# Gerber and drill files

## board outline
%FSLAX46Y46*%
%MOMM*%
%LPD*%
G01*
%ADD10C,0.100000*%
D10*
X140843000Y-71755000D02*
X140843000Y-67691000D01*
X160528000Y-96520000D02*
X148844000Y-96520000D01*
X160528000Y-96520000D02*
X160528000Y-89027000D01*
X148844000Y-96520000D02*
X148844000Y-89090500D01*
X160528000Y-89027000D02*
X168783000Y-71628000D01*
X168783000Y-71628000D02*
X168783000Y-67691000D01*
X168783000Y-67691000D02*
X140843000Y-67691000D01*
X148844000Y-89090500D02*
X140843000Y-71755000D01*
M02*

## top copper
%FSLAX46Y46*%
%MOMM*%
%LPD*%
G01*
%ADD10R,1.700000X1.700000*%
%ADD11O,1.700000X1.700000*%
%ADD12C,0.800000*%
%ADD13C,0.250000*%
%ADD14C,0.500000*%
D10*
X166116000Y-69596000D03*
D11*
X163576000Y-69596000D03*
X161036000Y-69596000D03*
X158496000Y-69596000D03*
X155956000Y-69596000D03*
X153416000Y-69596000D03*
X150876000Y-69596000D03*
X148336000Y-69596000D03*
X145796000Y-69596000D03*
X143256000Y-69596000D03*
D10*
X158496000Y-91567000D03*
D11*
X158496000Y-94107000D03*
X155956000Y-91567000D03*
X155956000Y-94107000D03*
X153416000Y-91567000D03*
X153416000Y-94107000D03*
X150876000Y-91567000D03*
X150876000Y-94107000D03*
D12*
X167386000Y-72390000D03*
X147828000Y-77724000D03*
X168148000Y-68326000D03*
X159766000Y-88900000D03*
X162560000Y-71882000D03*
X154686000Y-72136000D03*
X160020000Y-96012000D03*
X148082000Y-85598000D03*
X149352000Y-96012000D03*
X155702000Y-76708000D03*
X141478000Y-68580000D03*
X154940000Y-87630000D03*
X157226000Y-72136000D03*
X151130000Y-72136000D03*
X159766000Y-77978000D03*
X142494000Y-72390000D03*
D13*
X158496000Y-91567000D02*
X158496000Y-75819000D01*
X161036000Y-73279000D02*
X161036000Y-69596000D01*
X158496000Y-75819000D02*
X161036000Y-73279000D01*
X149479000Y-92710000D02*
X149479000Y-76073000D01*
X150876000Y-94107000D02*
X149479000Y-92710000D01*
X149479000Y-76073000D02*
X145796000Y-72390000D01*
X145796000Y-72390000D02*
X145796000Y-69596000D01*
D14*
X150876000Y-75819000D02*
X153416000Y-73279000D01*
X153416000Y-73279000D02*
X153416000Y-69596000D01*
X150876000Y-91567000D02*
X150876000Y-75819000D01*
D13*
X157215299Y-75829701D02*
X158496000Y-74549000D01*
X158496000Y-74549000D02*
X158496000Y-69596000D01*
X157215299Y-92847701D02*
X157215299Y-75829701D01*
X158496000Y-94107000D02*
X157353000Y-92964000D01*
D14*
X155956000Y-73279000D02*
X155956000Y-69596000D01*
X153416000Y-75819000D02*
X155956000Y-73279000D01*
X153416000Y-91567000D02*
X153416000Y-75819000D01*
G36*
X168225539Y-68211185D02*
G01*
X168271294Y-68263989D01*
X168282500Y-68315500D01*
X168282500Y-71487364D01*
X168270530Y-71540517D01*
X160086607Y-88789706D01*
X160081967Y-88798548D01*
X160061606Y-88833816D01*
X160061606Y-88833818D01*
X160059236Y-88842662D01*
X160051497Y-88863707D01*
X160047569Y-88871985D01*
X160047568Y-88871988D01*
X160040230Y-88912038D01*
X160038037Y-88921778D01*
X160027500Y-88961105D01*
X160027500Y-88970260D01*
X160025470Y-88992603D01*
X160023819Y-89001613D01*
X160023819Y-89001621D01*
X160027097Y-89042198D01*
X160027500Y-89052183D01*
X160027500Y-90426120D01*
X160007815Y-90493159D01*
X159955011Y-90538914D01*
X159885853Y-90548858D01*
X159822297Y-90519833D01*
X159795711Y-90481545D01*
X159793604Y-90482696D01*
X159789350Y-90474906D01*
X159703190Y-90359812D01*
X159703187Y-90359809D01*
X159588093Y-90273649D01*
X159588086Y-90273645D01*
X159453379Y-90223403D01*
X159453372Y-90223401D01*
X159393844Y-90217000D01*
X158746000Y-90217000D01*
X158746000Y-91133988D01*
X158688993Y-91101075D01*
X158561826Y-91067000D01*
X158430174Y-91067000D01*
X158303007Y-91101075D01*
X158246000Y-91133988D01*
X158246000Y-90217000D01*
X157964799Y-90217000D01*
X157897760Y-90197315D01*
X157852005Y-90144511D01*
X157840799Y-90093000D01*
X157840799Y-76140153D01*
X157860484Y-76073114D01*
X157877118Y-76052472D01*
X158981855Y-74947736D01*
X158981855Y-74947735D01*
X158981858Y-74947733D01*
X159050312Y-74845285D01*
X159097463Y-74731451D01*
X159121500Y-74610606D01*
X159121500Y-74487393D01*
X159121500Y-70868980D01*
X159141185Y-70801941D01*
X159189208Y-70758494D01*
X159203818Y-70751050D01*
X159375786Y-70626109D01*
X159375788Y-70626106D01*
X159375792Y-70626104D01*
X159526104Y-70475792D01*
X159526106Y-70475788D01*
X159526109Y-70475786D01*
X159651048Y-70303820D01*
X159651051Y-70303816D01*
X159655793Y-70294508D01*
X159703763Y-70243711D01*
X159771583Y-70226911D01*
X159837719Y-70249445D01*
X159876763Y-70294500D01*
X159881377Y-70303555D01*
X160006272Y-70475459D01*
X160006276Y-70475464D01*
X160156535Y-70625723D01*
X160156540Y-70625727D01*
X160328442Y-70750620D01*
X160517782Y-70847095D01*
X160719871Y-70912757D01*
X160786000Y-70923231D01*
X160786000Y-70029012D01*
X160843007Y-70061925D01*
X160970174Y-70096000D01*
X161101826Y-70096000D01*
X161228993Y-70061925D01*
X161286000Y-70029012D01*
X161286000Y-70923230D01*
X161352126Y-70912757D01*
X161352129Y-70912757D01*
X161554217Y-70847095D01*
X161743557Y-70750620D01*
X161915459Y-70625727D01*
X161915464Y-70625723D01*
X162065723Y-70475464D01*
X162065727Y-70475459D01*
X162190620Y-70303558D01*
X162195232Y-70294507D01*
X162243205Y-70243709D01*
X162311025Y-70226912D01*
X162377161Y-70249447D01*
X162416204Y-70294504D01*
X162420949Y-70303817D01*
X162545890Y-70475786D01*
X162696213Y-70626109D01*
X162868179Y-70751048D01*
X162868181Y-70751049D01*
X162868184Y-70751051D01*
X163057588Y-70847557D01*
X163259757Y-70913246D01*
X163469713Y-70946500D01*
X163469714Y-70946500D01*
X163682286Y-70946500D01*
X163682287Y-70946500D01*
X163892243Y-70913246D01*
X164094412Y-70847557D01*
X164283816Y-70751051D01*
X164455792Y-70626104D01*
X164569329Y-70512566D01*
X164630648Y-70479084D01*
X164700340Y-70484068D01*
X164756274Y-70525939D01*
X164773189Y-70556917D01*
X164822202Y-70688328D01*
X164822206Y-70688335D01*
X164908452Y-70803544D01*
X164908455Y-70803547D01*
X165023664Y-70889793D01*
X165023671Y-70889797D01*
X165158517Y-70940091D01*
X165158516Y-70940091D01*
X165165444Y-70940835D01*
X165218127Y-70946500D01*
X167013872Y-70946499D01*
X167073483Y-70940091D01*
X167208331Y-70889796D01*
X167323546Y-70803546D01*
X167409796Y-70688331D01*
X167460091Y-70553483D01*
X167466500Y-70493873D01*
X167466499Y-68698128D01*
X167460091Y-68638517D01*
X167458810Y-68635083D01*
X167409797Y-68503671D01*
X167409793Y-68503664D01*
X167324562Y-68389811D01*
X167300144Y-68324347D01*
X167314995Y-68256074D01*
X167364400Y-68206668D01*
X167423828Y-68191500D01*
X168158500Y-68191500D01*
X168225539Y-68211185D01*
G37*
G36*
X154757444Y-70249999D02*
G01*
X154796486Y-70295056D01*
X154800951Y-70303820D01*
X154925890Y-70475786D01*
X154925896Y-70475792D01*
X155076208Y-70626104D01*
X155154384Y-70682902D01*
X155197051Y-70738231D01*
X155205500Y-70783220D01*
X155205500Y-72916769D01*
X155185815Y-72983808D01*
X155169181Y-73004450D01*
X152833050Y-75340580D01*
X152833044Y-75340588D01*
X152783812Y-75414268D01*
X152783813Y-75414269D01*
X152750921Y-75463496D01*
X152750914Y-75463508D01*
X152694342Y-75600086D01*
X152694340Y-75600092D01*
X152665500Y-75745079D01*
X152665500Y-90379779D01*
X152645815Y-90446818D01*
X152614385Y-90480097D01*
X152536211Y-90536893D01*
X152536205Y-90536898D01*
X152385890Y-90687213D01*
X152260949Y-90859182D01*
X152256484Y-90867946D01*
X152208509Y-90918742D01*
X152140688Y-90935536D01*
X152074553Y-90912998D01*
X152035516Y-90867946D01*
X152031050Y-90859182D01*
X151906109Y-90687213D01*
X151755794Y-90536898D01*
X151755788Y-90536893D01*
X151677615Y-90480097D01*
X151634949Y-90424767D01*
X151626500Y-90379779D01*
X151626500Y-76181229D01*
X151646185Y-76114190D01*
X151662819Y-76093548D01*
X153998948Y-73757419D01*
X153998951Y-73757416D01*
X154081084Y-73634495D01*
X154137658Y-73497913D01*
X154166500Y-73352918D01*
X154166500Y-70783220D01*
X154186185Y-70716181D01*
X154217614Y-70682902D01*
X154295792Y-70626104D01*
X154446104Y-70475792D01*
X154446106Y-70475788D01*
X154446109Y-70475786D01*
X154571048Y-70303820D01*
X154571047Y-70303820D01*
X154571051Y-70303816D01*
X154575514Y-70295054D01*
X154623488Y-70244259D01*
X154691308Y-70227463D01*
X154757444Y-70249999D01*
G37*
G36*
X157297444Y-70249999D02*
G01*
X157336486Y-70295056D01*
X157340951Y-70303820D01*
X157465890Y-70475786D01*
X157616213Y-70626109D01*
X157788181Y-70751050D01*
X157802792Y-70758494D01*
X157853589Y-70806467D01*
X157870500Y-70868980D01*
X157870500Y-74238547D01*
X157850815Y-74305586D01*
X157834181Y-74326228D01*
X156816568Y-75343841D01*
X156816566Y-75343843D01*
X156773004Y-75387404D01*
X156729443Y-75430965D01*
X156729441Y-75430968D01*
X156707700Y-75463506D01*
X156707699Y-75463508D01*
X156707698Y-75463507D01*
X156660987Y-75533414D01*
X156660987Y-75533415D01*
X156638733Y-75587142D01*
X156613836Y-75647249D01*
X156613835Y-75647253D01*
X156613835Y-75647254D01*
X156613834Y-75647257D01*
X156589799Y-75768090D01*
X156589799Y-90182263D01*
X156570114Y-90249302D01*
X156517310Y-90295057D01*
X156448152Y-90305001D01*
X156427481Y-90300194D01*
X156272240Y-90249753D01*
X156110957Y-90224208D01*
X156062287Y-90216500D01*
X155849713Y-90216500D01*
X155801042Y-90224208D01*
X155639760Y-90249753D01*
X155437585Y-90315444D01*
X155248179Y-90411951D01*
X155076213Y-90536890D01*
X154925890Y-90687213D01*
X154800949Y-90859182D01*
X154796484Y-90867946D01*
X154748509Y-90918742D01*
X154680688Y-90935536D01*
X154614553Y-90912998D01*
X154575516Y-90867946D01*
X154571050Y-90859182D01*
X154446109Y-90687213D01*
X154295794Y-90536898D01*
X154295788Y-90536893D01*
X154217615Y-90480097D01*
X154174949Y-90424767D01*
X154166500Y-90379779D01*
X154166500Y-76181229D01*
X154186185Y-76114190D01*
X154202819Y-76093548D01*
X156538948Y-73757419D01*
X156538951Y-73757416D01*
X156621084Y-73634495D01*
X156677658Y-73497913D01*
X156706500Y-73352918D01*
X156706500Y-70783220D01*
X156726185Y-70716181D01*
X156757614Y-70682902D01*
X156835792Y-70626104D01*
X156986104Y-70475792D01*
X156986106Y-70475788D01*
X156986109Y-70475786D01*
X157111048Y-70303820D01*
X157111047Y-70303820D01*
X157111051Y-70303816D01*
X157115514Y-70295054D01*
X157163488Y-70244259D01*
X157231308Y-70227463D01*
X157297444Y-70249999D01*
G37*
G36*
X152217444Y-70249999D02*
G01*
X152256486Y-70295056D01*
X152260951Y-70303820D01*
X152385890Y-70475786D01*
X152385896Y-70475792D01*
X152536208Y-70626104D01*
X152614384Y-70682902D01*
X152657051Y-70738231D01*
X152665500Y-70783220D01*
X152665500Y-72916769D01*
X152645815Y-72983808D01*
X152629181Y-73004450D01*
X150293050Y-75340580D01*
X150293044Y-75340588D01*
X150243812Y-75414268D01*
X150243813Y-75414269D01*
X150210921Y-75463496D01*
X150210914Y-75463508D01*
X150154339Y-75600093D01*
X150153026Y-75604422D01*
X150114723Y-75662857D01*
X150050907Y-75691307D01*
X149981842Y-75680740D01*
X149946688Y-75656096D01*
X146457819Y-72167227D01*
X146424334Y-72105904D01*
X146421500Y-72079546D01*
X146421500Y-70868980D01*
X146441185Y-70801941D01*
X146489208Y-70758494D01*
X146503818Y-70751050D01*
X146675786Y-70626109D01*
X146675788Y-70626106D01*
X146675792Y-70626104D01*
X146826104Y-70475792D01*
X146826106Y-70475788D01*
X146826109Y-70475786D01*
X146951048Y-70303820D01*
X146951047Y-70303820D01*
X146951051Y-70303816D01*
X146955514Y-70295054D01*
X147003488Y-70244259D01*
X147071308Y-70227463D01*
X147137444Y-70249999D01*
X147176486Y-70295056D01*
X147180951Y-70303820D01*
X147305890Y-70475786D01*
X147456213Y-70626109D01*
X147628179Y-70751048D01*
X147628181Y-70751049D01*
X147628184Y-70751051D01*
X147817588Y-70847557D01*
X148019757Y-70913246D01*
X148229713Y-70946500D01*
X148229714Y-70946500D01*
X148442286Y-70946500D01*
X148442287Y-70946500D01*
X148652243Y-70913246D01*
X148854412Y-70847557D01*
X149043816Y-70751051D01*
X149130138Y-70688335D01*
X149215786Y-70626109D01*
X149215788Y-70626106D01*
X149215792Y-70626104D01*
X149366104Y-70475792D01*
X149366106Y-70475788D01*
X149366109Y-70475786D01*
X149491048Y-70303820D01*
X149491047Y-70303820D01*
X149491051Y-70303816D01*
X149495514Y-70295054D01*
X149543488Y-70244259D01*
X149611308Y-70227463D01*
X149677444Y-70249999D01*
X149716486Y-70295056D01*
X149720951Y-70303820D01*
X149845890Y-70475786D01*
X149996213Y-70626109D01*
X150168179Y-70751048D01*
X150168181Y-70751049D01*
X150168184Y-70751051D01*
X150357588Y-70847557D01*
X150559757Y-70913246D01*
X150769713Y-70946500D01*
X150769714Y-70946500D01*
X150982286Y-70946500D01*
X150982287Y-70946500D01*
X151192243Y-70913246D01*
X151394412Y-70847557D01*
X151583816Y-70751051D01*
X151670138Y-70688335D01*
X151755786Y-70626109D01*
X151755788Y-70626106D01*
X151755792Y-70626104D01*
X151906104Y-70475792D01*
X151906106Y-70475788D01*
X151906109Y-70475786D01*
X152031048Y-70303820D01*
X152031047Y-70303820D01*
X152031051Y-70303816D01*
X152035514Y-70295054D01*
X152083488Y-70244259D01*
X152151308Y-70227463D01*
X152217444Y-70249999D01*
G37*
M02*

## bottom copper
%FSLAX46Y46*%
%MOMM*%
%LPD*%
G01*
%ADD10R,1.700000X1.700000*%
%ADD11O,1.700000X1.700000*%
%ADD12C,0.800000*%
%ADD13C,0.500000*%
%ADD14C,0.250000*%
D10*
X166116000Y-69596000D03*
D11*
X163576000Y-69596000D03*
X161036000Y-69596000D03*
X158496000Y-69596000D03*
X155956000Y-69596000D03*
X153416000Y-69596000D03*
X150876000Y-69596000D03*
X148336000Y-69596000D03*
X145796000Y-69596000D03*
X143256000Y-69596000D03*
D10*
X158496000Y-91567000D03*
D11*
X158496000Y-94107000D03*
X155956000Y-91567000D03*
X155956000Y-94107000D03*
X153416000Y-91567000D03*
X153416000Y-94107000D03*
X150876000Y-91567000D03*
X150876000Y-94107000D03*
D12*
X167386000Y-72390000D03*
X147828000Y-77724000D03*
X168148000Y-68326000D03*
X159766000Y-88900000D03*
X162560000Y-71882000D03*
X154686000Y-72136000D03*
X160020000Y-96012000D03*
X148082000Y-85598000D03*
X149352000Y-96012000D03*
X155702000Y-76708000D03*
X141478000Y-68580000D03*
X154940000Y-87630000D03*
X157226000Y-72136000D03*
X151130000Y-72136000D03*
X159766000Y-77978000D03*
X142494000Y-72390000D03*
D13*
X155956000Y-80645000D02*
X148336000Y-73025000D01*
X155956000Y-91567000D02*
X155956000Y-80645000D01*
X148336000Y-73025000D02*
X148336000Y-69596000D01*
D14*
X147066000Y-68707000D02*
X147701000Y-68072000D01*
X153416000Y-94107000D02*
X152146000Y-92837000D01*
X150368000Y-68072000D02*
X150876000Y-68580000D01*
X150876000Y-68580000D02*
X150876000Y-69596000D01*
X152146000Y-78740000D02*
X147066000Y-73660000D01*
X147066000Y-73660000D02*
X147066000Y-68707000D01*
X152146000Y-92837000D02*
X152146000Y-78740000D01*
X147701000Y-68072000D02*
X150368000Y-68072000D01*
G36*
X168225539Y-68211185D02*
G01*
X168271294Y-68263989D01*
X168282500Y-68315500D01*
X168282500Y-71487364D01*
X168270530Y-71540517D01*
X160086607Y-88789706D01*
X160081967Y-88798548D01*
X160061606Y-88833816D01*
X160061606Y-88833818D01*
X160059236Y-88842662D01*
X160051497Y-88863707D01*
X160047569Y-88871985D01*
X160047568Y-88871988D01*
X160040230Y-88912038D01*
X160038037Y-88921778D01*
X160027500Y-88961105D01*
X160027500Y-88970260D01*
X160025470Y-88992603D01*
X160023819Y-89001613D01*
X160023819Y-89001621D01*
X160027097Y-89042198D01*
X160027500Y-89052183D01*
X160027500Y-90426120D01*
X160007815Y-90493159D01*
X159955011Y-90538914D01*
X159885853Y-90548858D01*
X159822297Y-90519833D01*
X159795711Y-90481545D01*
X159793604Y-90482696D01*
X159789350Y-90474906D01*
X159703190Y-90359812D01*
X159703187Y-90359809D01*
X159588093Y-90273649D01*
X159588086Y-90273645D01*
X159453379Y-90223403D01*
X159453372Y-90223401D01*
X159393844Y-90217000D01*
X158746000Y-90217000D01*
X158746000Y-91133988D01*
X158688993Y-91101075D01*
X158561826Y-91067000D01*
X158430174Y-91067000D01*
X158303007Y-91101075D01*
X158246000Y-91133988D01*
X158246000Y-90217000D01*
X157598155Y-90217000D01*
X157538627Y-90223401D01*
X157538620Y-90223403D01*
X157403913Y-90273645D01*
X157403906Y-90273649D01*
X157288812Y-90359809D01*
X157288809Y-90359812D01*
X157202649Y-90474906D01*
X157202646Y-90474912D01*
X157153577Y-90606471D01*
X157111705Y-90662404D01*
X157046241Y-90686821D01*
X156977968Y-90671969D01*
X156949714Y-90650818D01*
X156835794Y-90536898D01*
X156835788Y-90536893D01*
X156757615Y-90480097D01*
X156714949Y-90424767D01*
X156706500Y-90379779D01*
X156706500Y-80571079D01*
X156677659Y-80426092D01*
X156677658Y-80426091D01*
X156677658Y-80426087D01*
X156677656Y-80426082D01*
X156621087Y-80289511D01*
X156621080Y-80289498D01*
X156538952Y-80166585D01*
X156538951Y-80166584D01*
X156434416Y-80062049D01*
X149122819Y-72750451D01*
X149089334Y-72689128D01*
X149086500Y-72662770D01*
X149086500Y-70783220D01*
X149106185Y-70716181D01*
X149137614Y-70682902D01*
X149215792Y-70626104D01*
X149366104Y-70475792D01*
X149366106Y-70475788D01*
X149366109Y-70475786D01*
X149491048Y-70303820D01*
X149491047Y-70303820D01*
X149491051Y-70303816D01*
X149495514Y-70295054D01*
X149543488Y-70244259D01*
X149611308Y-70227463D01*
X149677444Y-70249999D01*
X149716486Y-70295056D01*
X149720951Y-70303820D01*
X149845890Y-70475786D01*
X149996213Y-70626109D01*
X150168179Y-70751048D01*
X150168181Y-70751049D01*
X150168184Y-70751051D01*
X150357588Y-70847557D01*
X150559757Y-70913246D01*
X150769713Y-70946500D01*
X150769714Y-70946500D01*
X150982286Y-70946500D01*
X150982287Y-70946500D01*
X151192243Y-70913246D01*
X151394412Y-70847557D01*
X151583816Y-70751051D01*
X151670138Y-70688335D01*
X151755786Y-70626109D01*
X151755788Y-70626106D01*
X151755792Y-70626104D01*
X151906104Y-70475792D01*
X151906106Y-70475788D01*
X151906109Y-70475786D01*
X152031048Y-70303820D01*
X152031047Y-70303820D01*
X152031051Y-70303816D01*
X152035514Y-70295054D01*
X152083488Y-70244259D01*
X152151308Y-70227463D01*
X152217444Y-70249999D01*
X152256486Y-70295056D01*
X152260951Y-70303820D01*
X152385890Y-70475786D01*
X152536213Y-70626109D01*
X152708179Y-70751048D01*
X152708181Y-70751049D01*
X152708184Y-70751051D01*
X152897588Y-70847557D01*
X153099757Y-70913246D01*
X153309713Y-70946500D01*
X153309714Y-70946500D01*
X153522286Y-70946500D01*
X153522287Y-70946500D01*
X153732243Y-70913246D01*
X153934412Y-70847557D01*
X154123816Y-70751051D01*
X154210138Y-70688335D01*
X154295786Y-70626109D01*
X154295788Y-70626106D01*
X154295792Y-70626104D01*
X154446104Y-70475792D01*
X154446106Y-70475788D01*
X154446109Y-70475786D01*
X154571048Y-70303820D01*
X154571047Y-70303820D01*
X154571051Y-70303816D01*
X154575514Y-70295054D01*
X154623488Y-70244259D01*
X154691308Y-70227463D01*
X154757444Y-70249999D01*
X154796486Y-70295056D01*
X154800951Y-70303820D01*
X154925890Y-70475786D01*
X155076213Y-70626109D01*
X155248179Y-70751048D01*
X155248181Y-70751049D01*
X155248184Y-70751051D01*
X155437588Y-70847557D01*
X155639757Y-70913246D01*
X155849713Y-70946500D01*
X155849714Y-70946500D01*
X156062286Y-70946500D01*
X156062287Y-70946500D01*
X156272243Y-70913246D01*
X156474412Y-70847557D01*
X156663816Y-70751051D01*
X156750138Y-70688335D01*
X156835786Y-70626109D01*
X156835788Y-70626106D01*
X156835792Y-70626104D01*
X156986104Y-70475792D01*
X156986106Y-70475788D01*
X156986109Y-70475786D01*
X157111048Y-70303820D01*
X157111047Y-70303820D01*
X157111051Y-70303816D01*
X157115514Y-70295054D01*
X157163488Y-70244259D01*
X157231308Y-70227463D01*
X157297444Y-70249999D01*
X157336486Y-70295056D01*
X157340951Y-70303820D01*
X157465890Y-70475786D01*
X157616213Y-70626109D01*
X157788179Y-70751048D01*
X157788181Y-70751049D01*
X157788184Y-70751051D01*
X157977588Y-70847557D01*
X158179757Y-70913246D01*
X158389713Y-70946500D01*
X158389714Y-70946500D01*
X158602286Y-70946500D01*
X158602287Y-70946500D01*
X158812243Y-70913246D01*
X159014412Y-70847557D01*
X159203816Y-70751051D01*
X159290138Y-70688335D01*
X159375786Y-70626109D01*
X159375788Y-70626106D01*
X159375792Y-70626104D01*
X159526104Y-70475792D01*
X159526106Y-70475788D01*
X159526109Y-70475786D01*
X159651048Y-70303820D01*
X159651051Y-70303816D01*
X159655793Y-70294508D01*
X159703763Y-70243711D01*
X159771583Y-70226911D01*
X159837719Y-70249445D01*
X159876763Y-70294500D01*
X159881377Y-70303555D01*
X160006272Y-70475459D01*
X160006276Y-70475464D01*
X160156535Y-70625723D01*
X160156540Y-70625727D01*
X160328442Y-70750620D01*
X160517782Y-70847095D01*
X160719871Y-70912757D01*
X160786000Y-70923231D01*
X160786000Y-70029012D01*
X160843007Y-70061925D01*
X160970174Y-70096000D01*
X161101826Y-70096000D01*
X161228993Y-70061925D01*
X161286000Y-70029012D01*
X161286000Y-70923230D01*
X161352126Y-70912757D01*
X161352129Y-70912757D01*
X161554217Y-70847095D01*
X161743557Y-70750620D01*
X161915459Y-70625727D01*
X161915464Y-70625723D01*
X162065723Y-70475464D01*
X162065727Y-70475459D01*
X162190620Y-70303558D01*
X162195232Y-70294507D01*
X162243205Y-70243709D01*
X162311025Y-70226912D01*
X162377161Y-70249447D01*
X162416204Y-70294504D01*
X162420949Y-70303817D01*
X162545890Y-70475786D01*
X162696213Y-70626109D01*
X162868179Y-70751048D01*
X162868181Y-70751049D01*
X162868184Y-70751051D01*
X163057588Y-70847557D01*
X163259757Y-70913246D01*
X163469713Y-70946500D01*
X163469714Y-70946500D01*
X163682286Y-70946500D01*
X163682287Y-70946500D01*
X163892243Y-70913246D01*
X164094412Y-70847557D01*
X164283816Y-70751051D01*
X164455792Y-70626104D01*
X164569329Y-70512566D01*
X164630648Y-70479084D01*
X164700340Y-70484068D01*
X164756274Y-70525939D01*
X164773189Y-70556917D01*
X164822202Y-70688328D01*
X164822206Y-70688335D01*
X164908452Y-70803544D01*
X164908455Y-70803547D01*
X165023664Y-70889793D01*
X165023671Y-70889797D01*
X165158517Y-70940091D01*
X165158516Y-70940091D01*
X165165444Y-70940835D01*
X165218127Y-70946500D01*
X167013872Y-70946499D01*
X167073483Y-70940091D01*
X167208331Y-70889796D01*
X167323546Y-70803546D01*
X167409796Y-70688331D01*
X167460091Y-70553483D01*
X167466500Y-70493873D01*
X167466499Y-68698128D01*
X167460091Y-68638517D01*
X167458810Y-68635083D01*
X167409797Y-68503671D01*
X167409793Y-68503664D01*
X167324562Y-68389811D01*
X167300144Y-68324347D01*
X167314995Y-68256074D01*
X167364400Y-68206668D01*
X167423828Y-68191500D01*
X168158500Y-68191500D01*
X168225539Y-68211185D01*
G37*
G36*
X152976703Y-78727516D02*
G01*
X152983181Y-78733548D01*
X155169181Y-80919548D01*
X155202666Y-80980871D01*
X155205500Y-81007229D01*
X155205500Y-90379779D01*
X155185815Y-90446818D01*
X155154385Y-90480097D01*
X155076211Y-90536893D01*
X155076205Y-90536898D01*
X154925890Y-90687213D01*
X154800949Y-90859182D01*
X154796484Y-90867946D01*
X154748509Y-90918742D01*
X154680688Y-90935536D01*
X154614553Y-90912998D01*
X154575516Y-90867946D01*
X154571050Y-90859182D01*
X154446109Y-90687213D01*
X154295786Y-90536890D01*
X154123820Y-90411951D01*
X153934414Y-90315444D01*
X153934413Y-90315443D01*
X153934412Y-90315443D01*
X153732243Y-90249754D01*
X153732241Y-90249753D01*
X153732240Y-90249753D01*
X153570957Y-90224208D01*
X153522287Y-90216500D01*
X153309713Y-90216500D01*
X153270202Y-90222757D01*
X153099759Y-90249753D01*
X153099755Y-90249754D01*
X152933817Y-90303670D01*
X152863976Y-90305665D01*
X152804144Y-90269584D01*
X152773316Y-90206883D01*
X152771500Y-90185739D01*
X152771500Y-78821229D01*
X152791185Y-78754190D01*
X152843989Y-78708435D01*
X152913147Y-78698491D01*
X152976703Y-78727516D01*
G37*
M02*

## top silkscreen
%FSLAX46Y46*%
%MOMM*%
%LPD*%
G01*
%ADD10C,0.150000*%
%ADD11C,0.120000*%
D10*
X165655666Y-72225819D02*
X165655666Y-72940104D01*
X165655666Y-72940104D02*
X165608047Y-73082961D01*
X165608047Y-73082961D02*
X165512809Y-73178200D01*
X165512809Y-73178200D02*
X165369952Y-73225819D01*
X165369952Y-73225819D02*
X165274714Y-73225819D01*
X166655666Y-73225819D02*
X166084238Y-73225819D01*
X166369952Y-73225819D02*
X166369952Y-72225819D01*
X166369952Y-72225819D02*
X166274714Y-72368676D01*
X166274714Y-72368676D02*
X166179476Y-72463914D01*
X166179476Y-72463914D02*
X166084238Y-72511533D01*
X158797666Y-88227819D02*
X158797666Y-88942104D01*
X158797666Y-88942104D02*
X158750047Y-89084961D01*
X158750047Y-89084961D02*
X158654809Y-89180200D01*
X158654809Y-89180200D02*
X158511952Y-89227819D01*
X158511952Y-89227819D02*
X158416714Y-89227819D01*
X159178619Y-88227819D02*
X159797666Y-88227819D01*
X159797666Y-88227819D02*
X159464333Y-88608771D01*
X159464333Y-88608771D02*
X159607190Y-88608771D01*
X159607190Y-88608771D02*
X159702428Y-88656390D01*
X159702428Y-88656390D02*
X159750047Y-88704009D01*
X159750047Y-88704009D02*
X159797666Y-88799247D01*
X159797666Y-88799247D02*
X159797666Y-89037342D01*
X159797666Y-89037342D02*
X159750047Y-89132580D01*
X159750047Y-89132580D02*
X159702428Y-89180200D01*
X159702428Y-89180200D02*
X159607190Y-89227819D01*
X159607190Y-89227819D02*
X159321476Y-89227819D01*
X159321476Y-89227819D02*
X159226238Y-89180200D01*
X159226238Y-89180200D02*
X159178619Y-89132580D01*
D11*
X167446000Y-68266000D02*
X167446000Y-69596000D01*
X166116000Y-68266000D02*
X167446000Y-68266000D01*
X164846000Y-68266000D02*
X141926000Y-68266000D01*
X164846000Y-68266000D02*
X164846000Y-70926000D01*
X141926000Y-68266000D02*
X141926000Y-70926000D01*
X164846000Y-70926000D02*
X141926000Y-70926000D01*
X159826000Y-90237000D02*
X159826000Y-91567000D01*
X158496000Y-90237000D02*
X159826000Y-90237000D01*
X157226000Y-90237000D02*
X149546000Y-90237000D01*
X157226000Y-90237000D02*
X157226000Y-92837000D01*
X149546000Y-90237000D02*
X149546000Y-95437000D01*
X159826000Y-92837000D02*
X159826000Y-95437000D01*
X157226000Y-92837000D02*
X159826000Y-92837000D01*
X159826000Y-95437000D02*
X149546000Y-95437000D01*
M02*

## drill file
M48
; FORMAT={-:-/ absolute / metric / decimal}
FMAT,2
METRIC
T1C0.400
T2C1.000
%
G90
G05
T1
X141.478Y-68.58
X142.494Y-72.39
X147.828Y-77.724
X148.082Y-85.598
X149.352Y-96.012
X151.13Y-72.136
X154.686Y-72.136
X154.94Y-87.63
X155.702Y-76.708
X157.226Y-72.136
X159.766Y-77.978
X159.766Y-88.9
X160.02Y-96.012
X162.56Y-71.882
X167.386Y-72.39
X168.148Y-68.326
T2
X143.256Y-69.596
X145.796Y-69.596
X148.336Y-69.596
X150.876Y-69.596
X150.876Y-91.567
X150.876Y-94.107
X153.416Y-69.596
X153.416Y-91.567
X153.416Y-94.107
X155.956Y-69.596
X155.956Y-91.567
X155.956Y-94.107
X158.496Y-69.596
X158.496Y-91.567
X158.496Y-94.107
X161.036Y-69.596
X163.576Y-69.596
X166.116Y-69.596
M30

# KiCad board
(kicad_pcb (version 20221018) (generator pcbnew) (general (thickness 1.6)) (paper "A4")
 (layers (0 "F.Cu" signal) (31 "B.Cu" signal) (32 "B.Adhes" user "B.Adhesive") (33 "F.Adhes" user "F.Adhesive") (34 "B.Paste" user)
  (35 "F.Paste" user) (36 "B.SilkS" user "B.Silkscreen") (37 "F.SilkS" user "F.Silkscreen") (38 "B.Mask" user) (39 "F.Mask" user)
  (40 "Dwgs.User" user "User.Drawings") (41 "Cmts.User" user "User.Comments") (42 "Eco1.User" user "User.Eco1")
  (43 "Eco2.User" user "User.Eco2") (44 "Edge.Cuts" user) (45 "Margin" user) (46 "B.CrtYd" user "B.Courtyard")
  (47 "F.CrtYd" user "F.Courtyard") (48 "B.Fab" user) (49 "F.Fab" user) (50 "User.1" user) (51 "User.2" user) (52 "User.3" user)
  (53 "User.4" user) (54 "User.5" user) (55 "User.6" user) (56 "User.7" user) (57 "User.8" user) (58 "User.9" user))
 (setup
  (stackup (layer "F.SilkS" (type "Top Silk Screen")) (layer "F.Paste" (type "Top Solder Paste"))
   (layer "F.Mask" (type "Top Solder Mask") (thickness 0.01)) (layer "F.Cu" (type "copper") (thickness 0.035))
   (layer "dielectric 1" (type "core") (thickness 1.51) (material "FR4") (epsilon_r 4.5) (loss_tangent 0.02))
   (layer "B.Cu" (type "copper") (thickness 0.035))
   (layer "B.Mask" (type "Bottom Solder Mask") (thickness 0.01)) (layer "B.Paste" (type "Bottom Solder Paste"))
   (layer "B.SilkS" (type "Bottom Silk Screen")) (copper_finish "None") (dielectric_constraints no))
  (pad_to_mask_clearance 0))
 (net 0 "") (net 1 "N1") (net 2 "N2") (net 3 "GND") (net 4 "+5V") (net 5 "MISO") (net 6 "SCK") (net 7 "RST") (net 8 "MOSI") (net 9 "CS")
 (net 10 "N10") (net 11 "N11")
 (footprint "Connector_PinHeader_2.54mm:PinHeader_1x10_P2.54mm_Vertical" (layer "F.Cu") (at 166.116 69.596 -90)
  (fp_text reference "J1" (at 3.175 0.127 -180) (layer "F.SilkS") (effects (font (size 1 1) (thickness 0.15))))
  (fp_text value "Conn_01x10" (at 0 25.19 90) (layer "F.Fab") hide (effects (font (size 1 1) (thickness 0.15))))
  (fp_line (start -1.33 -1.33) (end 0 -1.33) (stroke (width 0.12) (type solid)) (layer "F.SilkS"))
  (fp_line (start -1.33 0) (end -1.33 -1.33) (stroke (width 0.12) (type solid)) (layer "F.SilkS"))
  (fp_line (start -1.33 1.27) (end -1.33 24.19) (stroke (width 0.12) (type solid)) (layer "F.SilkS"))
  (fp_line (start -1.33 1.27) (end 1.33 1.27) (stroke (width 0.12) (type solid)) (layer "F.SilkS"))
  (fp_line (start -1.33 24.19) (end 1.33 24.19) (stroke (width 0.12) (type solid)) (layer "F.SilkS"))
  (fp_line (start 1.33 1.27) (end 1.33 24.19) (stroke (width 0.12) (type solid)) (layer "F.SilkS"))
  (pad "1" thru_hole rect (at 0 0 270) (size 1.7 1.7) (drill 1) (layers "*.Cu" "*.Mask") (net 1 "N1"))
  (pad "2" thru_hole oval (at 0 2.54 270) (size 1.7 1.7) (drill 1) (layers "*.Cu" "*.Mask") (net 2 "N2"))
  (pad "3" thru_hole oval (at 0 5.08 270) (size 1.7 1.7) (drill 1) (layers "*.Cu" "*.Mask") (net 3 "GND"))
  (pad "4" thru_hole oval (at 0 7.62 270) (size 1.7 1.7) (drill 1) (layers "*.Cu" "*.Mask") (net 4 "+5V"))
  (pad "5" thru_hole oval (at 0 10.16 270) (size 1.7 1.7) (drill 1) (layers "*.Cu" "*.Mask") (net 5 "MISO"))
  (pad "6" thru_hole oval (at 0 12.7 270) (size 1.7 1.7) (drill 1) (layers "*.Cu" "*.Mask") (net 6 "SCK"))
  (pad "7" thru_hole oval (at 0 15.24 270) (size 1.7 1.7) (drill 1) (layers "*.Cu" "*.Mask") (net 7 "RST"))
  (pad "8" thru_hole oval (at 0 17.78 270) (size 1.7 1.7) (drill 1) (layers "*.Cu" "*.Mask") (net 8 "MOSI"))
  (pad "9" thru_hole oval (at 0 20.32 270) (size 1.7 1.7) (drill 1) (layers "*.Cu" "*.Mask") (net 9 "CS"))
  (pad "10" thru_hole oval (at 0 22.86 270) (size 1.7 1.7) (drill 1) (layers "*.Cu" "*.Mask") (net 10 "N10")))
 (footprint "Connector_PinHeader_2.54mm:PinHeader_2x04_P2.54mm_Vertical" (layer "F.Cu") (at 158.496 91.567 -90)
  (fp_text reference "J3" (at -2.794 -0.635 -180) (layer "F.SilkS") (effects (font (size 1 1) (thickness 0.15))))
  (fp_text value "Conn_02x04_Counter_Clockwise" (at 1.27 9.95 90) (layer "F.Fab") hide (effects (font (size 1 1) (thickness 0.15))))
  (fp_line (start -1.33 -1.33) (end 0 -1.33) (stroke (width 0.12) (type solid)) (layer "F.SilkS"))
  (fp_line (start -1.33 0) (end -1.33 -1.33) (stroke (width 0.12) (type solid)) (layer "F.SilkS"))
  (fp_line (start -1.33 1.27) (end -1.33 8.95) (stroke (width 0.12) (type solid)) (layer "F.SilkS"))
  (fp_line (start -1.33 1.27) (end 1.27 1.27) (stroke (width 0.12) (type solid)) (layer "F.SilkS"))
  (fp_line (start -1.33 8.95) (end 3.87 8.95) (stroke (width 0.12) (type solid)) (layer "F.SilkS"))
  (fp_line (start 1.27 -1.33) (end 3.87 -1.33) (stroke (width 0.12) (type solid)) (layer "F.SilkS"))
  (fp_line (start 1.27 1.27) (end 1.27 -1.33) (stroke (width 0.12) (type solid)) (layer "F.SilkS"))
  (fp_line (start 3.87 -1.33) (end 3.87 8.95) (stroke (width 0.12) (type solid)) (layer "F.SilkS"))
  (pad "1" thru_hole rect (at 0 0 270) (size 1.7 1.7) (drill 1) (layers "*.Cu" "*.Mask") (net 3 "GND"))
  (pad "2" thru_hole oval (at 2.54 0 270) (size 1.7 1.7) (drill 1) (layers "*.Cu" "*.Mask") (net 4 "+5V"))
  (pad "3" thru_hole oval (at 0 2.54 270) (size 1.7 1.7) (drill 1) (layers "*.Cu" "*.Mask") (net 8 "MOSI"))
  (pad "4" thru_hole oval (at 2.54 2.54 270) (size 1.7 1.7) (drill 1) (layers "*.Cu" "*.Mask") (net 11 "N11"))
  (pad "5" thru_hole oval (at 0 5.08 270) (size 1.7 1.7) (drill 1) (layers "*.Cu" "*.Mask") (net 5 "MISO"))
  (pad "6" thru_hole oval (at 2.54 5.08 270) (size 1.7 1.7) (drill 1) (layers "*.Cu" "*.Mask") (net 7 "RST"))
  (pad "7" thru_hole oval (at 0 7.62 270) (size 1.7 1.7) (drill 1) (layers "*.Cu" "*.Mask") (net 6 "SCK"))
  (pad "8" thru_hole oval (at 2.54 7.62 270) (size 1.7 1.7) (drill 1) (layers "*.Cu" "*.Mask") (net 9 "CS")))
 (gr_line (start 140.843 71.755) (end 140.843 67.691) (stroke (width 0.1) (type default)) (layer "Edge.Cuts"))
 (gr_line (start 160.528 96.52) (end 148.844 96.52) (stroke (width 0.1) (type default)) (layer "Edge.Cuts"))
 (gr_line (start 160.528 96.52) (end 160.528 89.027) (stroke (width 0.1) (type default)) (layer "Edge.Cuts"))
 (gr_line (start 148.844 96.52) (end 148.844 89.0905) (stroke (width 0.1) (type default)) (layer "Edge.Cuts"))
 (gr_line (start 160.528 89.027) (end 168.783 71.628) (stroke (width 0.1) (type default)) (layer "Edge.Cuts"))
 (gr_line (start 168.783 71.628) (end 168.783 67.691) (stroke (width 0.1) (type default)) (layer "Edge.Cuts"))
 (gr_line (start 168.783 67.691) (end 140.843 67.691) (stroke (width 0.1) (type default)) (layer "Edge.Cuts"))
 (gr_line (start 148.844 89.0905) (end 140.843 71.755) (stroke (width 0.1) (type default)) (layer "Edge.Cuts"))
 (segment (start 158.496 91.567) (end 158.496 75.819) (width 0.25) (layer "F.Cu") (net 3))
 (segment (start 161.036 73.279) (end 161.036 69.596) (width 0.25) (layer "F.Cu") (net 3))
 (segment (start 158.496 75.819) (end 161.036 73.279) (width 0.25) (layer "F.Cu") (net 3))
 (via (at 167.386 72.39) (size 0.8) (drill 0.4) (layers "F.Cu" "B.Cu") (free) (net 3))
 (via (at 147.828 77.724) (size 0.8) (drill 0.4) (layers "F.Cu" "B.Cu") (free) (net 3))
 (via (at 168.148 68.326) (size 0.8) (drill 0.4) (layers "F.Cu" "B.Cu") (free) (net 3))
 (via (at 159.766 88.9) (size 0.8) (drill 0.4) (layers "F.Cu" "B.Cu") (free) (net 3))
 (via (at 162.56 71.882) (size 0.8) (drill 0.4) (layers "F.Cu" "B.Cu") (free) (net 3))
 (via (at 154.686 72.136) (size 0.8) (drill 0.4) (layers "F.Cu" "B.Cu") (free) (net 3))
 (via (at 160.02 96.012) (size 0.8) (drill 0.4) (layers "F.Cu" "B.Cu") (free) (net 3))
 (via (at 148.082 85.598) (size 0.8) (drill 0.4) (layers "F.Cu" "B.Cu") (free) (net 3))
 (via (at 149.352 96.012) (size 0.8) (drill 0.4) (layers "F.Cu" "B.Cu") (free) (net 3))
 (via (at 155.702 76.708) (size 0.8) (drill 0.4) (layers "F.Cu" "B.Cu") (free) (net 3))
 (via (at 141.478 68.58) (size 0.8) (drill 0.4) (layers "F.Cu" "B.Cu") (free) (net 3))
 (via (at 154.94 87.63) (size 0.8) (drill 0.4) (layers "F.Cu" "B.Cu") (free) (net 3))
 (via (at 157.226 72.136) (size 0.8) (drill 0.4) (layers "F.Cu" "B.Cu") (free) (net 3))
 (via (at 151.13 72.136) (size 0.8) (drill 0.4) (layers "F.Cu" "B.Cu") (free) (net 3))
 (via (at 159.766 77.978) (size 0.8) (drill 0.4) (layers "F.Cu" "B.Cu") (free) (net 3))
 (via (at 142.494 72.39) (size 0.8) (drill 0.4) (layers "F.Cu" "B.Cu") (free) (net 3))
 (segment (start 149.479 92.71) (end 149.479 76.073) (width 0.25) (layer "F.Cu") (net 9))
 (segment (start 150.876 94.107) (end 149.479 92.71) (width 0.25) (layer "F.Cu") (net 9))
 (segment (start 149.479 76.073) (end 145.796 72.39) (width 0.25) (layer "F.Cu") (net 9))
 (segment (start 145.796 72.39) (end 145.796 69.596) (width 0.25) (layer "F.Cu") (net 9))
 (segment (start 155.956 80.645) (end 148.336 73.025) (width 0.5) (layer "B.Cu") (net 8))
 (segment (start 155.956 91.567) (end 155.956 80.645) (width 0.5) (layer "B.Cu") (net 8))
 (segment (start 148.336 73.025) (end 148.336 69.596) (width 0.5) (layer "B.Cu") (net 8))
 (segment (start 150.876 75.819) (end 153.416 73.279) (width 0.5) (layer "F.Cu") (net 6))
 (segment (start 153.416 73.279) (end 153.416 69.596) (width 0.5) (layer "F.Cu") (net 6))
 (segment (start 150.876 91.567) (end 150.876 75.819) (width 0.5) (layer "F.Cu") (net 6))
 (segment (start 157.215299 75.829701) (end 158.496 74.549) (width 0.25) (layer "F.Cu") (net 4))
 (segment (start 158.496 74.549) (end 158.496 69.596) (width 0.25) (layer "F.Cu") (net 4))
 (segment (start 157.215299 92.847701) (end 157.215299 75.829701) (width 0.25) (layer "F.Cu") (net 4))
 (segment (start 158.496 94.107) (end 157.353 92.964) (width 0.25) (layer "F.Cu") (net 4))
 (segment (start 155.956 73.279) (end 155.956 69.596) (width 0.5) (layer "F.Cu") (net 5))
 (segment (start 153.416 75.819) (end 155.956 73.279) (width 0.5) (layer "F.Cu") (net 5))
 (segment (start 153.416 91.567) (end 153.416 75.819) (width 0.5) (layer "F.Cu") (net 5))
 (segment (start 147.066 68.707) (end 147.701 68.072) (width 0.25) (layer "B.Cu") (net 7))
 (segment (start 153.416 94.107) (end 152.146 92.837) (width 0.25) (layer "B.Cu") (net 7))
 (segment (start 150.368 68.072) (end 150.876 68.58) (width 0.25) (layer "B.Cu") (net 7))
 (segment (start 150.876 68.58) (end 150.876 69.596) (width 0.25) (layer "B.Cu") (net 7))
 (segment (start 152.146 78.74) (end 147.066 73.66) (width 0.25) (layer "B.Cu") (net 7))
 (segment (start 147.066 73.66) (end 147.066 68.707) (width 0.25) (layer "B.Cu") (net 7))
 (segment (start 152.146 92.837) (end 152.146 78.74) (width 0.25) (layer "B.Cu") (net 7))
 (segment (start 147.701 68.072) (end 150.368 68.072) (width 0.25) (layer "B.Cu") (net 7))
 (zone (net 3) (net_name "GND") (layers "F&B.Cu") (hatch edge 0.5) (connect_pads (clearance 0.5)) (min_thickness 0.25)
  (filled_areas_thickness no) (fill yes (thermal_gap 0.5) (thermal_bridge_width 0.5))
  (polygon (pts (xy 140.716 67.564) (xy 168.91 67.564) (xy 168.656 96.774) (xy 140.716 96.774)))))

